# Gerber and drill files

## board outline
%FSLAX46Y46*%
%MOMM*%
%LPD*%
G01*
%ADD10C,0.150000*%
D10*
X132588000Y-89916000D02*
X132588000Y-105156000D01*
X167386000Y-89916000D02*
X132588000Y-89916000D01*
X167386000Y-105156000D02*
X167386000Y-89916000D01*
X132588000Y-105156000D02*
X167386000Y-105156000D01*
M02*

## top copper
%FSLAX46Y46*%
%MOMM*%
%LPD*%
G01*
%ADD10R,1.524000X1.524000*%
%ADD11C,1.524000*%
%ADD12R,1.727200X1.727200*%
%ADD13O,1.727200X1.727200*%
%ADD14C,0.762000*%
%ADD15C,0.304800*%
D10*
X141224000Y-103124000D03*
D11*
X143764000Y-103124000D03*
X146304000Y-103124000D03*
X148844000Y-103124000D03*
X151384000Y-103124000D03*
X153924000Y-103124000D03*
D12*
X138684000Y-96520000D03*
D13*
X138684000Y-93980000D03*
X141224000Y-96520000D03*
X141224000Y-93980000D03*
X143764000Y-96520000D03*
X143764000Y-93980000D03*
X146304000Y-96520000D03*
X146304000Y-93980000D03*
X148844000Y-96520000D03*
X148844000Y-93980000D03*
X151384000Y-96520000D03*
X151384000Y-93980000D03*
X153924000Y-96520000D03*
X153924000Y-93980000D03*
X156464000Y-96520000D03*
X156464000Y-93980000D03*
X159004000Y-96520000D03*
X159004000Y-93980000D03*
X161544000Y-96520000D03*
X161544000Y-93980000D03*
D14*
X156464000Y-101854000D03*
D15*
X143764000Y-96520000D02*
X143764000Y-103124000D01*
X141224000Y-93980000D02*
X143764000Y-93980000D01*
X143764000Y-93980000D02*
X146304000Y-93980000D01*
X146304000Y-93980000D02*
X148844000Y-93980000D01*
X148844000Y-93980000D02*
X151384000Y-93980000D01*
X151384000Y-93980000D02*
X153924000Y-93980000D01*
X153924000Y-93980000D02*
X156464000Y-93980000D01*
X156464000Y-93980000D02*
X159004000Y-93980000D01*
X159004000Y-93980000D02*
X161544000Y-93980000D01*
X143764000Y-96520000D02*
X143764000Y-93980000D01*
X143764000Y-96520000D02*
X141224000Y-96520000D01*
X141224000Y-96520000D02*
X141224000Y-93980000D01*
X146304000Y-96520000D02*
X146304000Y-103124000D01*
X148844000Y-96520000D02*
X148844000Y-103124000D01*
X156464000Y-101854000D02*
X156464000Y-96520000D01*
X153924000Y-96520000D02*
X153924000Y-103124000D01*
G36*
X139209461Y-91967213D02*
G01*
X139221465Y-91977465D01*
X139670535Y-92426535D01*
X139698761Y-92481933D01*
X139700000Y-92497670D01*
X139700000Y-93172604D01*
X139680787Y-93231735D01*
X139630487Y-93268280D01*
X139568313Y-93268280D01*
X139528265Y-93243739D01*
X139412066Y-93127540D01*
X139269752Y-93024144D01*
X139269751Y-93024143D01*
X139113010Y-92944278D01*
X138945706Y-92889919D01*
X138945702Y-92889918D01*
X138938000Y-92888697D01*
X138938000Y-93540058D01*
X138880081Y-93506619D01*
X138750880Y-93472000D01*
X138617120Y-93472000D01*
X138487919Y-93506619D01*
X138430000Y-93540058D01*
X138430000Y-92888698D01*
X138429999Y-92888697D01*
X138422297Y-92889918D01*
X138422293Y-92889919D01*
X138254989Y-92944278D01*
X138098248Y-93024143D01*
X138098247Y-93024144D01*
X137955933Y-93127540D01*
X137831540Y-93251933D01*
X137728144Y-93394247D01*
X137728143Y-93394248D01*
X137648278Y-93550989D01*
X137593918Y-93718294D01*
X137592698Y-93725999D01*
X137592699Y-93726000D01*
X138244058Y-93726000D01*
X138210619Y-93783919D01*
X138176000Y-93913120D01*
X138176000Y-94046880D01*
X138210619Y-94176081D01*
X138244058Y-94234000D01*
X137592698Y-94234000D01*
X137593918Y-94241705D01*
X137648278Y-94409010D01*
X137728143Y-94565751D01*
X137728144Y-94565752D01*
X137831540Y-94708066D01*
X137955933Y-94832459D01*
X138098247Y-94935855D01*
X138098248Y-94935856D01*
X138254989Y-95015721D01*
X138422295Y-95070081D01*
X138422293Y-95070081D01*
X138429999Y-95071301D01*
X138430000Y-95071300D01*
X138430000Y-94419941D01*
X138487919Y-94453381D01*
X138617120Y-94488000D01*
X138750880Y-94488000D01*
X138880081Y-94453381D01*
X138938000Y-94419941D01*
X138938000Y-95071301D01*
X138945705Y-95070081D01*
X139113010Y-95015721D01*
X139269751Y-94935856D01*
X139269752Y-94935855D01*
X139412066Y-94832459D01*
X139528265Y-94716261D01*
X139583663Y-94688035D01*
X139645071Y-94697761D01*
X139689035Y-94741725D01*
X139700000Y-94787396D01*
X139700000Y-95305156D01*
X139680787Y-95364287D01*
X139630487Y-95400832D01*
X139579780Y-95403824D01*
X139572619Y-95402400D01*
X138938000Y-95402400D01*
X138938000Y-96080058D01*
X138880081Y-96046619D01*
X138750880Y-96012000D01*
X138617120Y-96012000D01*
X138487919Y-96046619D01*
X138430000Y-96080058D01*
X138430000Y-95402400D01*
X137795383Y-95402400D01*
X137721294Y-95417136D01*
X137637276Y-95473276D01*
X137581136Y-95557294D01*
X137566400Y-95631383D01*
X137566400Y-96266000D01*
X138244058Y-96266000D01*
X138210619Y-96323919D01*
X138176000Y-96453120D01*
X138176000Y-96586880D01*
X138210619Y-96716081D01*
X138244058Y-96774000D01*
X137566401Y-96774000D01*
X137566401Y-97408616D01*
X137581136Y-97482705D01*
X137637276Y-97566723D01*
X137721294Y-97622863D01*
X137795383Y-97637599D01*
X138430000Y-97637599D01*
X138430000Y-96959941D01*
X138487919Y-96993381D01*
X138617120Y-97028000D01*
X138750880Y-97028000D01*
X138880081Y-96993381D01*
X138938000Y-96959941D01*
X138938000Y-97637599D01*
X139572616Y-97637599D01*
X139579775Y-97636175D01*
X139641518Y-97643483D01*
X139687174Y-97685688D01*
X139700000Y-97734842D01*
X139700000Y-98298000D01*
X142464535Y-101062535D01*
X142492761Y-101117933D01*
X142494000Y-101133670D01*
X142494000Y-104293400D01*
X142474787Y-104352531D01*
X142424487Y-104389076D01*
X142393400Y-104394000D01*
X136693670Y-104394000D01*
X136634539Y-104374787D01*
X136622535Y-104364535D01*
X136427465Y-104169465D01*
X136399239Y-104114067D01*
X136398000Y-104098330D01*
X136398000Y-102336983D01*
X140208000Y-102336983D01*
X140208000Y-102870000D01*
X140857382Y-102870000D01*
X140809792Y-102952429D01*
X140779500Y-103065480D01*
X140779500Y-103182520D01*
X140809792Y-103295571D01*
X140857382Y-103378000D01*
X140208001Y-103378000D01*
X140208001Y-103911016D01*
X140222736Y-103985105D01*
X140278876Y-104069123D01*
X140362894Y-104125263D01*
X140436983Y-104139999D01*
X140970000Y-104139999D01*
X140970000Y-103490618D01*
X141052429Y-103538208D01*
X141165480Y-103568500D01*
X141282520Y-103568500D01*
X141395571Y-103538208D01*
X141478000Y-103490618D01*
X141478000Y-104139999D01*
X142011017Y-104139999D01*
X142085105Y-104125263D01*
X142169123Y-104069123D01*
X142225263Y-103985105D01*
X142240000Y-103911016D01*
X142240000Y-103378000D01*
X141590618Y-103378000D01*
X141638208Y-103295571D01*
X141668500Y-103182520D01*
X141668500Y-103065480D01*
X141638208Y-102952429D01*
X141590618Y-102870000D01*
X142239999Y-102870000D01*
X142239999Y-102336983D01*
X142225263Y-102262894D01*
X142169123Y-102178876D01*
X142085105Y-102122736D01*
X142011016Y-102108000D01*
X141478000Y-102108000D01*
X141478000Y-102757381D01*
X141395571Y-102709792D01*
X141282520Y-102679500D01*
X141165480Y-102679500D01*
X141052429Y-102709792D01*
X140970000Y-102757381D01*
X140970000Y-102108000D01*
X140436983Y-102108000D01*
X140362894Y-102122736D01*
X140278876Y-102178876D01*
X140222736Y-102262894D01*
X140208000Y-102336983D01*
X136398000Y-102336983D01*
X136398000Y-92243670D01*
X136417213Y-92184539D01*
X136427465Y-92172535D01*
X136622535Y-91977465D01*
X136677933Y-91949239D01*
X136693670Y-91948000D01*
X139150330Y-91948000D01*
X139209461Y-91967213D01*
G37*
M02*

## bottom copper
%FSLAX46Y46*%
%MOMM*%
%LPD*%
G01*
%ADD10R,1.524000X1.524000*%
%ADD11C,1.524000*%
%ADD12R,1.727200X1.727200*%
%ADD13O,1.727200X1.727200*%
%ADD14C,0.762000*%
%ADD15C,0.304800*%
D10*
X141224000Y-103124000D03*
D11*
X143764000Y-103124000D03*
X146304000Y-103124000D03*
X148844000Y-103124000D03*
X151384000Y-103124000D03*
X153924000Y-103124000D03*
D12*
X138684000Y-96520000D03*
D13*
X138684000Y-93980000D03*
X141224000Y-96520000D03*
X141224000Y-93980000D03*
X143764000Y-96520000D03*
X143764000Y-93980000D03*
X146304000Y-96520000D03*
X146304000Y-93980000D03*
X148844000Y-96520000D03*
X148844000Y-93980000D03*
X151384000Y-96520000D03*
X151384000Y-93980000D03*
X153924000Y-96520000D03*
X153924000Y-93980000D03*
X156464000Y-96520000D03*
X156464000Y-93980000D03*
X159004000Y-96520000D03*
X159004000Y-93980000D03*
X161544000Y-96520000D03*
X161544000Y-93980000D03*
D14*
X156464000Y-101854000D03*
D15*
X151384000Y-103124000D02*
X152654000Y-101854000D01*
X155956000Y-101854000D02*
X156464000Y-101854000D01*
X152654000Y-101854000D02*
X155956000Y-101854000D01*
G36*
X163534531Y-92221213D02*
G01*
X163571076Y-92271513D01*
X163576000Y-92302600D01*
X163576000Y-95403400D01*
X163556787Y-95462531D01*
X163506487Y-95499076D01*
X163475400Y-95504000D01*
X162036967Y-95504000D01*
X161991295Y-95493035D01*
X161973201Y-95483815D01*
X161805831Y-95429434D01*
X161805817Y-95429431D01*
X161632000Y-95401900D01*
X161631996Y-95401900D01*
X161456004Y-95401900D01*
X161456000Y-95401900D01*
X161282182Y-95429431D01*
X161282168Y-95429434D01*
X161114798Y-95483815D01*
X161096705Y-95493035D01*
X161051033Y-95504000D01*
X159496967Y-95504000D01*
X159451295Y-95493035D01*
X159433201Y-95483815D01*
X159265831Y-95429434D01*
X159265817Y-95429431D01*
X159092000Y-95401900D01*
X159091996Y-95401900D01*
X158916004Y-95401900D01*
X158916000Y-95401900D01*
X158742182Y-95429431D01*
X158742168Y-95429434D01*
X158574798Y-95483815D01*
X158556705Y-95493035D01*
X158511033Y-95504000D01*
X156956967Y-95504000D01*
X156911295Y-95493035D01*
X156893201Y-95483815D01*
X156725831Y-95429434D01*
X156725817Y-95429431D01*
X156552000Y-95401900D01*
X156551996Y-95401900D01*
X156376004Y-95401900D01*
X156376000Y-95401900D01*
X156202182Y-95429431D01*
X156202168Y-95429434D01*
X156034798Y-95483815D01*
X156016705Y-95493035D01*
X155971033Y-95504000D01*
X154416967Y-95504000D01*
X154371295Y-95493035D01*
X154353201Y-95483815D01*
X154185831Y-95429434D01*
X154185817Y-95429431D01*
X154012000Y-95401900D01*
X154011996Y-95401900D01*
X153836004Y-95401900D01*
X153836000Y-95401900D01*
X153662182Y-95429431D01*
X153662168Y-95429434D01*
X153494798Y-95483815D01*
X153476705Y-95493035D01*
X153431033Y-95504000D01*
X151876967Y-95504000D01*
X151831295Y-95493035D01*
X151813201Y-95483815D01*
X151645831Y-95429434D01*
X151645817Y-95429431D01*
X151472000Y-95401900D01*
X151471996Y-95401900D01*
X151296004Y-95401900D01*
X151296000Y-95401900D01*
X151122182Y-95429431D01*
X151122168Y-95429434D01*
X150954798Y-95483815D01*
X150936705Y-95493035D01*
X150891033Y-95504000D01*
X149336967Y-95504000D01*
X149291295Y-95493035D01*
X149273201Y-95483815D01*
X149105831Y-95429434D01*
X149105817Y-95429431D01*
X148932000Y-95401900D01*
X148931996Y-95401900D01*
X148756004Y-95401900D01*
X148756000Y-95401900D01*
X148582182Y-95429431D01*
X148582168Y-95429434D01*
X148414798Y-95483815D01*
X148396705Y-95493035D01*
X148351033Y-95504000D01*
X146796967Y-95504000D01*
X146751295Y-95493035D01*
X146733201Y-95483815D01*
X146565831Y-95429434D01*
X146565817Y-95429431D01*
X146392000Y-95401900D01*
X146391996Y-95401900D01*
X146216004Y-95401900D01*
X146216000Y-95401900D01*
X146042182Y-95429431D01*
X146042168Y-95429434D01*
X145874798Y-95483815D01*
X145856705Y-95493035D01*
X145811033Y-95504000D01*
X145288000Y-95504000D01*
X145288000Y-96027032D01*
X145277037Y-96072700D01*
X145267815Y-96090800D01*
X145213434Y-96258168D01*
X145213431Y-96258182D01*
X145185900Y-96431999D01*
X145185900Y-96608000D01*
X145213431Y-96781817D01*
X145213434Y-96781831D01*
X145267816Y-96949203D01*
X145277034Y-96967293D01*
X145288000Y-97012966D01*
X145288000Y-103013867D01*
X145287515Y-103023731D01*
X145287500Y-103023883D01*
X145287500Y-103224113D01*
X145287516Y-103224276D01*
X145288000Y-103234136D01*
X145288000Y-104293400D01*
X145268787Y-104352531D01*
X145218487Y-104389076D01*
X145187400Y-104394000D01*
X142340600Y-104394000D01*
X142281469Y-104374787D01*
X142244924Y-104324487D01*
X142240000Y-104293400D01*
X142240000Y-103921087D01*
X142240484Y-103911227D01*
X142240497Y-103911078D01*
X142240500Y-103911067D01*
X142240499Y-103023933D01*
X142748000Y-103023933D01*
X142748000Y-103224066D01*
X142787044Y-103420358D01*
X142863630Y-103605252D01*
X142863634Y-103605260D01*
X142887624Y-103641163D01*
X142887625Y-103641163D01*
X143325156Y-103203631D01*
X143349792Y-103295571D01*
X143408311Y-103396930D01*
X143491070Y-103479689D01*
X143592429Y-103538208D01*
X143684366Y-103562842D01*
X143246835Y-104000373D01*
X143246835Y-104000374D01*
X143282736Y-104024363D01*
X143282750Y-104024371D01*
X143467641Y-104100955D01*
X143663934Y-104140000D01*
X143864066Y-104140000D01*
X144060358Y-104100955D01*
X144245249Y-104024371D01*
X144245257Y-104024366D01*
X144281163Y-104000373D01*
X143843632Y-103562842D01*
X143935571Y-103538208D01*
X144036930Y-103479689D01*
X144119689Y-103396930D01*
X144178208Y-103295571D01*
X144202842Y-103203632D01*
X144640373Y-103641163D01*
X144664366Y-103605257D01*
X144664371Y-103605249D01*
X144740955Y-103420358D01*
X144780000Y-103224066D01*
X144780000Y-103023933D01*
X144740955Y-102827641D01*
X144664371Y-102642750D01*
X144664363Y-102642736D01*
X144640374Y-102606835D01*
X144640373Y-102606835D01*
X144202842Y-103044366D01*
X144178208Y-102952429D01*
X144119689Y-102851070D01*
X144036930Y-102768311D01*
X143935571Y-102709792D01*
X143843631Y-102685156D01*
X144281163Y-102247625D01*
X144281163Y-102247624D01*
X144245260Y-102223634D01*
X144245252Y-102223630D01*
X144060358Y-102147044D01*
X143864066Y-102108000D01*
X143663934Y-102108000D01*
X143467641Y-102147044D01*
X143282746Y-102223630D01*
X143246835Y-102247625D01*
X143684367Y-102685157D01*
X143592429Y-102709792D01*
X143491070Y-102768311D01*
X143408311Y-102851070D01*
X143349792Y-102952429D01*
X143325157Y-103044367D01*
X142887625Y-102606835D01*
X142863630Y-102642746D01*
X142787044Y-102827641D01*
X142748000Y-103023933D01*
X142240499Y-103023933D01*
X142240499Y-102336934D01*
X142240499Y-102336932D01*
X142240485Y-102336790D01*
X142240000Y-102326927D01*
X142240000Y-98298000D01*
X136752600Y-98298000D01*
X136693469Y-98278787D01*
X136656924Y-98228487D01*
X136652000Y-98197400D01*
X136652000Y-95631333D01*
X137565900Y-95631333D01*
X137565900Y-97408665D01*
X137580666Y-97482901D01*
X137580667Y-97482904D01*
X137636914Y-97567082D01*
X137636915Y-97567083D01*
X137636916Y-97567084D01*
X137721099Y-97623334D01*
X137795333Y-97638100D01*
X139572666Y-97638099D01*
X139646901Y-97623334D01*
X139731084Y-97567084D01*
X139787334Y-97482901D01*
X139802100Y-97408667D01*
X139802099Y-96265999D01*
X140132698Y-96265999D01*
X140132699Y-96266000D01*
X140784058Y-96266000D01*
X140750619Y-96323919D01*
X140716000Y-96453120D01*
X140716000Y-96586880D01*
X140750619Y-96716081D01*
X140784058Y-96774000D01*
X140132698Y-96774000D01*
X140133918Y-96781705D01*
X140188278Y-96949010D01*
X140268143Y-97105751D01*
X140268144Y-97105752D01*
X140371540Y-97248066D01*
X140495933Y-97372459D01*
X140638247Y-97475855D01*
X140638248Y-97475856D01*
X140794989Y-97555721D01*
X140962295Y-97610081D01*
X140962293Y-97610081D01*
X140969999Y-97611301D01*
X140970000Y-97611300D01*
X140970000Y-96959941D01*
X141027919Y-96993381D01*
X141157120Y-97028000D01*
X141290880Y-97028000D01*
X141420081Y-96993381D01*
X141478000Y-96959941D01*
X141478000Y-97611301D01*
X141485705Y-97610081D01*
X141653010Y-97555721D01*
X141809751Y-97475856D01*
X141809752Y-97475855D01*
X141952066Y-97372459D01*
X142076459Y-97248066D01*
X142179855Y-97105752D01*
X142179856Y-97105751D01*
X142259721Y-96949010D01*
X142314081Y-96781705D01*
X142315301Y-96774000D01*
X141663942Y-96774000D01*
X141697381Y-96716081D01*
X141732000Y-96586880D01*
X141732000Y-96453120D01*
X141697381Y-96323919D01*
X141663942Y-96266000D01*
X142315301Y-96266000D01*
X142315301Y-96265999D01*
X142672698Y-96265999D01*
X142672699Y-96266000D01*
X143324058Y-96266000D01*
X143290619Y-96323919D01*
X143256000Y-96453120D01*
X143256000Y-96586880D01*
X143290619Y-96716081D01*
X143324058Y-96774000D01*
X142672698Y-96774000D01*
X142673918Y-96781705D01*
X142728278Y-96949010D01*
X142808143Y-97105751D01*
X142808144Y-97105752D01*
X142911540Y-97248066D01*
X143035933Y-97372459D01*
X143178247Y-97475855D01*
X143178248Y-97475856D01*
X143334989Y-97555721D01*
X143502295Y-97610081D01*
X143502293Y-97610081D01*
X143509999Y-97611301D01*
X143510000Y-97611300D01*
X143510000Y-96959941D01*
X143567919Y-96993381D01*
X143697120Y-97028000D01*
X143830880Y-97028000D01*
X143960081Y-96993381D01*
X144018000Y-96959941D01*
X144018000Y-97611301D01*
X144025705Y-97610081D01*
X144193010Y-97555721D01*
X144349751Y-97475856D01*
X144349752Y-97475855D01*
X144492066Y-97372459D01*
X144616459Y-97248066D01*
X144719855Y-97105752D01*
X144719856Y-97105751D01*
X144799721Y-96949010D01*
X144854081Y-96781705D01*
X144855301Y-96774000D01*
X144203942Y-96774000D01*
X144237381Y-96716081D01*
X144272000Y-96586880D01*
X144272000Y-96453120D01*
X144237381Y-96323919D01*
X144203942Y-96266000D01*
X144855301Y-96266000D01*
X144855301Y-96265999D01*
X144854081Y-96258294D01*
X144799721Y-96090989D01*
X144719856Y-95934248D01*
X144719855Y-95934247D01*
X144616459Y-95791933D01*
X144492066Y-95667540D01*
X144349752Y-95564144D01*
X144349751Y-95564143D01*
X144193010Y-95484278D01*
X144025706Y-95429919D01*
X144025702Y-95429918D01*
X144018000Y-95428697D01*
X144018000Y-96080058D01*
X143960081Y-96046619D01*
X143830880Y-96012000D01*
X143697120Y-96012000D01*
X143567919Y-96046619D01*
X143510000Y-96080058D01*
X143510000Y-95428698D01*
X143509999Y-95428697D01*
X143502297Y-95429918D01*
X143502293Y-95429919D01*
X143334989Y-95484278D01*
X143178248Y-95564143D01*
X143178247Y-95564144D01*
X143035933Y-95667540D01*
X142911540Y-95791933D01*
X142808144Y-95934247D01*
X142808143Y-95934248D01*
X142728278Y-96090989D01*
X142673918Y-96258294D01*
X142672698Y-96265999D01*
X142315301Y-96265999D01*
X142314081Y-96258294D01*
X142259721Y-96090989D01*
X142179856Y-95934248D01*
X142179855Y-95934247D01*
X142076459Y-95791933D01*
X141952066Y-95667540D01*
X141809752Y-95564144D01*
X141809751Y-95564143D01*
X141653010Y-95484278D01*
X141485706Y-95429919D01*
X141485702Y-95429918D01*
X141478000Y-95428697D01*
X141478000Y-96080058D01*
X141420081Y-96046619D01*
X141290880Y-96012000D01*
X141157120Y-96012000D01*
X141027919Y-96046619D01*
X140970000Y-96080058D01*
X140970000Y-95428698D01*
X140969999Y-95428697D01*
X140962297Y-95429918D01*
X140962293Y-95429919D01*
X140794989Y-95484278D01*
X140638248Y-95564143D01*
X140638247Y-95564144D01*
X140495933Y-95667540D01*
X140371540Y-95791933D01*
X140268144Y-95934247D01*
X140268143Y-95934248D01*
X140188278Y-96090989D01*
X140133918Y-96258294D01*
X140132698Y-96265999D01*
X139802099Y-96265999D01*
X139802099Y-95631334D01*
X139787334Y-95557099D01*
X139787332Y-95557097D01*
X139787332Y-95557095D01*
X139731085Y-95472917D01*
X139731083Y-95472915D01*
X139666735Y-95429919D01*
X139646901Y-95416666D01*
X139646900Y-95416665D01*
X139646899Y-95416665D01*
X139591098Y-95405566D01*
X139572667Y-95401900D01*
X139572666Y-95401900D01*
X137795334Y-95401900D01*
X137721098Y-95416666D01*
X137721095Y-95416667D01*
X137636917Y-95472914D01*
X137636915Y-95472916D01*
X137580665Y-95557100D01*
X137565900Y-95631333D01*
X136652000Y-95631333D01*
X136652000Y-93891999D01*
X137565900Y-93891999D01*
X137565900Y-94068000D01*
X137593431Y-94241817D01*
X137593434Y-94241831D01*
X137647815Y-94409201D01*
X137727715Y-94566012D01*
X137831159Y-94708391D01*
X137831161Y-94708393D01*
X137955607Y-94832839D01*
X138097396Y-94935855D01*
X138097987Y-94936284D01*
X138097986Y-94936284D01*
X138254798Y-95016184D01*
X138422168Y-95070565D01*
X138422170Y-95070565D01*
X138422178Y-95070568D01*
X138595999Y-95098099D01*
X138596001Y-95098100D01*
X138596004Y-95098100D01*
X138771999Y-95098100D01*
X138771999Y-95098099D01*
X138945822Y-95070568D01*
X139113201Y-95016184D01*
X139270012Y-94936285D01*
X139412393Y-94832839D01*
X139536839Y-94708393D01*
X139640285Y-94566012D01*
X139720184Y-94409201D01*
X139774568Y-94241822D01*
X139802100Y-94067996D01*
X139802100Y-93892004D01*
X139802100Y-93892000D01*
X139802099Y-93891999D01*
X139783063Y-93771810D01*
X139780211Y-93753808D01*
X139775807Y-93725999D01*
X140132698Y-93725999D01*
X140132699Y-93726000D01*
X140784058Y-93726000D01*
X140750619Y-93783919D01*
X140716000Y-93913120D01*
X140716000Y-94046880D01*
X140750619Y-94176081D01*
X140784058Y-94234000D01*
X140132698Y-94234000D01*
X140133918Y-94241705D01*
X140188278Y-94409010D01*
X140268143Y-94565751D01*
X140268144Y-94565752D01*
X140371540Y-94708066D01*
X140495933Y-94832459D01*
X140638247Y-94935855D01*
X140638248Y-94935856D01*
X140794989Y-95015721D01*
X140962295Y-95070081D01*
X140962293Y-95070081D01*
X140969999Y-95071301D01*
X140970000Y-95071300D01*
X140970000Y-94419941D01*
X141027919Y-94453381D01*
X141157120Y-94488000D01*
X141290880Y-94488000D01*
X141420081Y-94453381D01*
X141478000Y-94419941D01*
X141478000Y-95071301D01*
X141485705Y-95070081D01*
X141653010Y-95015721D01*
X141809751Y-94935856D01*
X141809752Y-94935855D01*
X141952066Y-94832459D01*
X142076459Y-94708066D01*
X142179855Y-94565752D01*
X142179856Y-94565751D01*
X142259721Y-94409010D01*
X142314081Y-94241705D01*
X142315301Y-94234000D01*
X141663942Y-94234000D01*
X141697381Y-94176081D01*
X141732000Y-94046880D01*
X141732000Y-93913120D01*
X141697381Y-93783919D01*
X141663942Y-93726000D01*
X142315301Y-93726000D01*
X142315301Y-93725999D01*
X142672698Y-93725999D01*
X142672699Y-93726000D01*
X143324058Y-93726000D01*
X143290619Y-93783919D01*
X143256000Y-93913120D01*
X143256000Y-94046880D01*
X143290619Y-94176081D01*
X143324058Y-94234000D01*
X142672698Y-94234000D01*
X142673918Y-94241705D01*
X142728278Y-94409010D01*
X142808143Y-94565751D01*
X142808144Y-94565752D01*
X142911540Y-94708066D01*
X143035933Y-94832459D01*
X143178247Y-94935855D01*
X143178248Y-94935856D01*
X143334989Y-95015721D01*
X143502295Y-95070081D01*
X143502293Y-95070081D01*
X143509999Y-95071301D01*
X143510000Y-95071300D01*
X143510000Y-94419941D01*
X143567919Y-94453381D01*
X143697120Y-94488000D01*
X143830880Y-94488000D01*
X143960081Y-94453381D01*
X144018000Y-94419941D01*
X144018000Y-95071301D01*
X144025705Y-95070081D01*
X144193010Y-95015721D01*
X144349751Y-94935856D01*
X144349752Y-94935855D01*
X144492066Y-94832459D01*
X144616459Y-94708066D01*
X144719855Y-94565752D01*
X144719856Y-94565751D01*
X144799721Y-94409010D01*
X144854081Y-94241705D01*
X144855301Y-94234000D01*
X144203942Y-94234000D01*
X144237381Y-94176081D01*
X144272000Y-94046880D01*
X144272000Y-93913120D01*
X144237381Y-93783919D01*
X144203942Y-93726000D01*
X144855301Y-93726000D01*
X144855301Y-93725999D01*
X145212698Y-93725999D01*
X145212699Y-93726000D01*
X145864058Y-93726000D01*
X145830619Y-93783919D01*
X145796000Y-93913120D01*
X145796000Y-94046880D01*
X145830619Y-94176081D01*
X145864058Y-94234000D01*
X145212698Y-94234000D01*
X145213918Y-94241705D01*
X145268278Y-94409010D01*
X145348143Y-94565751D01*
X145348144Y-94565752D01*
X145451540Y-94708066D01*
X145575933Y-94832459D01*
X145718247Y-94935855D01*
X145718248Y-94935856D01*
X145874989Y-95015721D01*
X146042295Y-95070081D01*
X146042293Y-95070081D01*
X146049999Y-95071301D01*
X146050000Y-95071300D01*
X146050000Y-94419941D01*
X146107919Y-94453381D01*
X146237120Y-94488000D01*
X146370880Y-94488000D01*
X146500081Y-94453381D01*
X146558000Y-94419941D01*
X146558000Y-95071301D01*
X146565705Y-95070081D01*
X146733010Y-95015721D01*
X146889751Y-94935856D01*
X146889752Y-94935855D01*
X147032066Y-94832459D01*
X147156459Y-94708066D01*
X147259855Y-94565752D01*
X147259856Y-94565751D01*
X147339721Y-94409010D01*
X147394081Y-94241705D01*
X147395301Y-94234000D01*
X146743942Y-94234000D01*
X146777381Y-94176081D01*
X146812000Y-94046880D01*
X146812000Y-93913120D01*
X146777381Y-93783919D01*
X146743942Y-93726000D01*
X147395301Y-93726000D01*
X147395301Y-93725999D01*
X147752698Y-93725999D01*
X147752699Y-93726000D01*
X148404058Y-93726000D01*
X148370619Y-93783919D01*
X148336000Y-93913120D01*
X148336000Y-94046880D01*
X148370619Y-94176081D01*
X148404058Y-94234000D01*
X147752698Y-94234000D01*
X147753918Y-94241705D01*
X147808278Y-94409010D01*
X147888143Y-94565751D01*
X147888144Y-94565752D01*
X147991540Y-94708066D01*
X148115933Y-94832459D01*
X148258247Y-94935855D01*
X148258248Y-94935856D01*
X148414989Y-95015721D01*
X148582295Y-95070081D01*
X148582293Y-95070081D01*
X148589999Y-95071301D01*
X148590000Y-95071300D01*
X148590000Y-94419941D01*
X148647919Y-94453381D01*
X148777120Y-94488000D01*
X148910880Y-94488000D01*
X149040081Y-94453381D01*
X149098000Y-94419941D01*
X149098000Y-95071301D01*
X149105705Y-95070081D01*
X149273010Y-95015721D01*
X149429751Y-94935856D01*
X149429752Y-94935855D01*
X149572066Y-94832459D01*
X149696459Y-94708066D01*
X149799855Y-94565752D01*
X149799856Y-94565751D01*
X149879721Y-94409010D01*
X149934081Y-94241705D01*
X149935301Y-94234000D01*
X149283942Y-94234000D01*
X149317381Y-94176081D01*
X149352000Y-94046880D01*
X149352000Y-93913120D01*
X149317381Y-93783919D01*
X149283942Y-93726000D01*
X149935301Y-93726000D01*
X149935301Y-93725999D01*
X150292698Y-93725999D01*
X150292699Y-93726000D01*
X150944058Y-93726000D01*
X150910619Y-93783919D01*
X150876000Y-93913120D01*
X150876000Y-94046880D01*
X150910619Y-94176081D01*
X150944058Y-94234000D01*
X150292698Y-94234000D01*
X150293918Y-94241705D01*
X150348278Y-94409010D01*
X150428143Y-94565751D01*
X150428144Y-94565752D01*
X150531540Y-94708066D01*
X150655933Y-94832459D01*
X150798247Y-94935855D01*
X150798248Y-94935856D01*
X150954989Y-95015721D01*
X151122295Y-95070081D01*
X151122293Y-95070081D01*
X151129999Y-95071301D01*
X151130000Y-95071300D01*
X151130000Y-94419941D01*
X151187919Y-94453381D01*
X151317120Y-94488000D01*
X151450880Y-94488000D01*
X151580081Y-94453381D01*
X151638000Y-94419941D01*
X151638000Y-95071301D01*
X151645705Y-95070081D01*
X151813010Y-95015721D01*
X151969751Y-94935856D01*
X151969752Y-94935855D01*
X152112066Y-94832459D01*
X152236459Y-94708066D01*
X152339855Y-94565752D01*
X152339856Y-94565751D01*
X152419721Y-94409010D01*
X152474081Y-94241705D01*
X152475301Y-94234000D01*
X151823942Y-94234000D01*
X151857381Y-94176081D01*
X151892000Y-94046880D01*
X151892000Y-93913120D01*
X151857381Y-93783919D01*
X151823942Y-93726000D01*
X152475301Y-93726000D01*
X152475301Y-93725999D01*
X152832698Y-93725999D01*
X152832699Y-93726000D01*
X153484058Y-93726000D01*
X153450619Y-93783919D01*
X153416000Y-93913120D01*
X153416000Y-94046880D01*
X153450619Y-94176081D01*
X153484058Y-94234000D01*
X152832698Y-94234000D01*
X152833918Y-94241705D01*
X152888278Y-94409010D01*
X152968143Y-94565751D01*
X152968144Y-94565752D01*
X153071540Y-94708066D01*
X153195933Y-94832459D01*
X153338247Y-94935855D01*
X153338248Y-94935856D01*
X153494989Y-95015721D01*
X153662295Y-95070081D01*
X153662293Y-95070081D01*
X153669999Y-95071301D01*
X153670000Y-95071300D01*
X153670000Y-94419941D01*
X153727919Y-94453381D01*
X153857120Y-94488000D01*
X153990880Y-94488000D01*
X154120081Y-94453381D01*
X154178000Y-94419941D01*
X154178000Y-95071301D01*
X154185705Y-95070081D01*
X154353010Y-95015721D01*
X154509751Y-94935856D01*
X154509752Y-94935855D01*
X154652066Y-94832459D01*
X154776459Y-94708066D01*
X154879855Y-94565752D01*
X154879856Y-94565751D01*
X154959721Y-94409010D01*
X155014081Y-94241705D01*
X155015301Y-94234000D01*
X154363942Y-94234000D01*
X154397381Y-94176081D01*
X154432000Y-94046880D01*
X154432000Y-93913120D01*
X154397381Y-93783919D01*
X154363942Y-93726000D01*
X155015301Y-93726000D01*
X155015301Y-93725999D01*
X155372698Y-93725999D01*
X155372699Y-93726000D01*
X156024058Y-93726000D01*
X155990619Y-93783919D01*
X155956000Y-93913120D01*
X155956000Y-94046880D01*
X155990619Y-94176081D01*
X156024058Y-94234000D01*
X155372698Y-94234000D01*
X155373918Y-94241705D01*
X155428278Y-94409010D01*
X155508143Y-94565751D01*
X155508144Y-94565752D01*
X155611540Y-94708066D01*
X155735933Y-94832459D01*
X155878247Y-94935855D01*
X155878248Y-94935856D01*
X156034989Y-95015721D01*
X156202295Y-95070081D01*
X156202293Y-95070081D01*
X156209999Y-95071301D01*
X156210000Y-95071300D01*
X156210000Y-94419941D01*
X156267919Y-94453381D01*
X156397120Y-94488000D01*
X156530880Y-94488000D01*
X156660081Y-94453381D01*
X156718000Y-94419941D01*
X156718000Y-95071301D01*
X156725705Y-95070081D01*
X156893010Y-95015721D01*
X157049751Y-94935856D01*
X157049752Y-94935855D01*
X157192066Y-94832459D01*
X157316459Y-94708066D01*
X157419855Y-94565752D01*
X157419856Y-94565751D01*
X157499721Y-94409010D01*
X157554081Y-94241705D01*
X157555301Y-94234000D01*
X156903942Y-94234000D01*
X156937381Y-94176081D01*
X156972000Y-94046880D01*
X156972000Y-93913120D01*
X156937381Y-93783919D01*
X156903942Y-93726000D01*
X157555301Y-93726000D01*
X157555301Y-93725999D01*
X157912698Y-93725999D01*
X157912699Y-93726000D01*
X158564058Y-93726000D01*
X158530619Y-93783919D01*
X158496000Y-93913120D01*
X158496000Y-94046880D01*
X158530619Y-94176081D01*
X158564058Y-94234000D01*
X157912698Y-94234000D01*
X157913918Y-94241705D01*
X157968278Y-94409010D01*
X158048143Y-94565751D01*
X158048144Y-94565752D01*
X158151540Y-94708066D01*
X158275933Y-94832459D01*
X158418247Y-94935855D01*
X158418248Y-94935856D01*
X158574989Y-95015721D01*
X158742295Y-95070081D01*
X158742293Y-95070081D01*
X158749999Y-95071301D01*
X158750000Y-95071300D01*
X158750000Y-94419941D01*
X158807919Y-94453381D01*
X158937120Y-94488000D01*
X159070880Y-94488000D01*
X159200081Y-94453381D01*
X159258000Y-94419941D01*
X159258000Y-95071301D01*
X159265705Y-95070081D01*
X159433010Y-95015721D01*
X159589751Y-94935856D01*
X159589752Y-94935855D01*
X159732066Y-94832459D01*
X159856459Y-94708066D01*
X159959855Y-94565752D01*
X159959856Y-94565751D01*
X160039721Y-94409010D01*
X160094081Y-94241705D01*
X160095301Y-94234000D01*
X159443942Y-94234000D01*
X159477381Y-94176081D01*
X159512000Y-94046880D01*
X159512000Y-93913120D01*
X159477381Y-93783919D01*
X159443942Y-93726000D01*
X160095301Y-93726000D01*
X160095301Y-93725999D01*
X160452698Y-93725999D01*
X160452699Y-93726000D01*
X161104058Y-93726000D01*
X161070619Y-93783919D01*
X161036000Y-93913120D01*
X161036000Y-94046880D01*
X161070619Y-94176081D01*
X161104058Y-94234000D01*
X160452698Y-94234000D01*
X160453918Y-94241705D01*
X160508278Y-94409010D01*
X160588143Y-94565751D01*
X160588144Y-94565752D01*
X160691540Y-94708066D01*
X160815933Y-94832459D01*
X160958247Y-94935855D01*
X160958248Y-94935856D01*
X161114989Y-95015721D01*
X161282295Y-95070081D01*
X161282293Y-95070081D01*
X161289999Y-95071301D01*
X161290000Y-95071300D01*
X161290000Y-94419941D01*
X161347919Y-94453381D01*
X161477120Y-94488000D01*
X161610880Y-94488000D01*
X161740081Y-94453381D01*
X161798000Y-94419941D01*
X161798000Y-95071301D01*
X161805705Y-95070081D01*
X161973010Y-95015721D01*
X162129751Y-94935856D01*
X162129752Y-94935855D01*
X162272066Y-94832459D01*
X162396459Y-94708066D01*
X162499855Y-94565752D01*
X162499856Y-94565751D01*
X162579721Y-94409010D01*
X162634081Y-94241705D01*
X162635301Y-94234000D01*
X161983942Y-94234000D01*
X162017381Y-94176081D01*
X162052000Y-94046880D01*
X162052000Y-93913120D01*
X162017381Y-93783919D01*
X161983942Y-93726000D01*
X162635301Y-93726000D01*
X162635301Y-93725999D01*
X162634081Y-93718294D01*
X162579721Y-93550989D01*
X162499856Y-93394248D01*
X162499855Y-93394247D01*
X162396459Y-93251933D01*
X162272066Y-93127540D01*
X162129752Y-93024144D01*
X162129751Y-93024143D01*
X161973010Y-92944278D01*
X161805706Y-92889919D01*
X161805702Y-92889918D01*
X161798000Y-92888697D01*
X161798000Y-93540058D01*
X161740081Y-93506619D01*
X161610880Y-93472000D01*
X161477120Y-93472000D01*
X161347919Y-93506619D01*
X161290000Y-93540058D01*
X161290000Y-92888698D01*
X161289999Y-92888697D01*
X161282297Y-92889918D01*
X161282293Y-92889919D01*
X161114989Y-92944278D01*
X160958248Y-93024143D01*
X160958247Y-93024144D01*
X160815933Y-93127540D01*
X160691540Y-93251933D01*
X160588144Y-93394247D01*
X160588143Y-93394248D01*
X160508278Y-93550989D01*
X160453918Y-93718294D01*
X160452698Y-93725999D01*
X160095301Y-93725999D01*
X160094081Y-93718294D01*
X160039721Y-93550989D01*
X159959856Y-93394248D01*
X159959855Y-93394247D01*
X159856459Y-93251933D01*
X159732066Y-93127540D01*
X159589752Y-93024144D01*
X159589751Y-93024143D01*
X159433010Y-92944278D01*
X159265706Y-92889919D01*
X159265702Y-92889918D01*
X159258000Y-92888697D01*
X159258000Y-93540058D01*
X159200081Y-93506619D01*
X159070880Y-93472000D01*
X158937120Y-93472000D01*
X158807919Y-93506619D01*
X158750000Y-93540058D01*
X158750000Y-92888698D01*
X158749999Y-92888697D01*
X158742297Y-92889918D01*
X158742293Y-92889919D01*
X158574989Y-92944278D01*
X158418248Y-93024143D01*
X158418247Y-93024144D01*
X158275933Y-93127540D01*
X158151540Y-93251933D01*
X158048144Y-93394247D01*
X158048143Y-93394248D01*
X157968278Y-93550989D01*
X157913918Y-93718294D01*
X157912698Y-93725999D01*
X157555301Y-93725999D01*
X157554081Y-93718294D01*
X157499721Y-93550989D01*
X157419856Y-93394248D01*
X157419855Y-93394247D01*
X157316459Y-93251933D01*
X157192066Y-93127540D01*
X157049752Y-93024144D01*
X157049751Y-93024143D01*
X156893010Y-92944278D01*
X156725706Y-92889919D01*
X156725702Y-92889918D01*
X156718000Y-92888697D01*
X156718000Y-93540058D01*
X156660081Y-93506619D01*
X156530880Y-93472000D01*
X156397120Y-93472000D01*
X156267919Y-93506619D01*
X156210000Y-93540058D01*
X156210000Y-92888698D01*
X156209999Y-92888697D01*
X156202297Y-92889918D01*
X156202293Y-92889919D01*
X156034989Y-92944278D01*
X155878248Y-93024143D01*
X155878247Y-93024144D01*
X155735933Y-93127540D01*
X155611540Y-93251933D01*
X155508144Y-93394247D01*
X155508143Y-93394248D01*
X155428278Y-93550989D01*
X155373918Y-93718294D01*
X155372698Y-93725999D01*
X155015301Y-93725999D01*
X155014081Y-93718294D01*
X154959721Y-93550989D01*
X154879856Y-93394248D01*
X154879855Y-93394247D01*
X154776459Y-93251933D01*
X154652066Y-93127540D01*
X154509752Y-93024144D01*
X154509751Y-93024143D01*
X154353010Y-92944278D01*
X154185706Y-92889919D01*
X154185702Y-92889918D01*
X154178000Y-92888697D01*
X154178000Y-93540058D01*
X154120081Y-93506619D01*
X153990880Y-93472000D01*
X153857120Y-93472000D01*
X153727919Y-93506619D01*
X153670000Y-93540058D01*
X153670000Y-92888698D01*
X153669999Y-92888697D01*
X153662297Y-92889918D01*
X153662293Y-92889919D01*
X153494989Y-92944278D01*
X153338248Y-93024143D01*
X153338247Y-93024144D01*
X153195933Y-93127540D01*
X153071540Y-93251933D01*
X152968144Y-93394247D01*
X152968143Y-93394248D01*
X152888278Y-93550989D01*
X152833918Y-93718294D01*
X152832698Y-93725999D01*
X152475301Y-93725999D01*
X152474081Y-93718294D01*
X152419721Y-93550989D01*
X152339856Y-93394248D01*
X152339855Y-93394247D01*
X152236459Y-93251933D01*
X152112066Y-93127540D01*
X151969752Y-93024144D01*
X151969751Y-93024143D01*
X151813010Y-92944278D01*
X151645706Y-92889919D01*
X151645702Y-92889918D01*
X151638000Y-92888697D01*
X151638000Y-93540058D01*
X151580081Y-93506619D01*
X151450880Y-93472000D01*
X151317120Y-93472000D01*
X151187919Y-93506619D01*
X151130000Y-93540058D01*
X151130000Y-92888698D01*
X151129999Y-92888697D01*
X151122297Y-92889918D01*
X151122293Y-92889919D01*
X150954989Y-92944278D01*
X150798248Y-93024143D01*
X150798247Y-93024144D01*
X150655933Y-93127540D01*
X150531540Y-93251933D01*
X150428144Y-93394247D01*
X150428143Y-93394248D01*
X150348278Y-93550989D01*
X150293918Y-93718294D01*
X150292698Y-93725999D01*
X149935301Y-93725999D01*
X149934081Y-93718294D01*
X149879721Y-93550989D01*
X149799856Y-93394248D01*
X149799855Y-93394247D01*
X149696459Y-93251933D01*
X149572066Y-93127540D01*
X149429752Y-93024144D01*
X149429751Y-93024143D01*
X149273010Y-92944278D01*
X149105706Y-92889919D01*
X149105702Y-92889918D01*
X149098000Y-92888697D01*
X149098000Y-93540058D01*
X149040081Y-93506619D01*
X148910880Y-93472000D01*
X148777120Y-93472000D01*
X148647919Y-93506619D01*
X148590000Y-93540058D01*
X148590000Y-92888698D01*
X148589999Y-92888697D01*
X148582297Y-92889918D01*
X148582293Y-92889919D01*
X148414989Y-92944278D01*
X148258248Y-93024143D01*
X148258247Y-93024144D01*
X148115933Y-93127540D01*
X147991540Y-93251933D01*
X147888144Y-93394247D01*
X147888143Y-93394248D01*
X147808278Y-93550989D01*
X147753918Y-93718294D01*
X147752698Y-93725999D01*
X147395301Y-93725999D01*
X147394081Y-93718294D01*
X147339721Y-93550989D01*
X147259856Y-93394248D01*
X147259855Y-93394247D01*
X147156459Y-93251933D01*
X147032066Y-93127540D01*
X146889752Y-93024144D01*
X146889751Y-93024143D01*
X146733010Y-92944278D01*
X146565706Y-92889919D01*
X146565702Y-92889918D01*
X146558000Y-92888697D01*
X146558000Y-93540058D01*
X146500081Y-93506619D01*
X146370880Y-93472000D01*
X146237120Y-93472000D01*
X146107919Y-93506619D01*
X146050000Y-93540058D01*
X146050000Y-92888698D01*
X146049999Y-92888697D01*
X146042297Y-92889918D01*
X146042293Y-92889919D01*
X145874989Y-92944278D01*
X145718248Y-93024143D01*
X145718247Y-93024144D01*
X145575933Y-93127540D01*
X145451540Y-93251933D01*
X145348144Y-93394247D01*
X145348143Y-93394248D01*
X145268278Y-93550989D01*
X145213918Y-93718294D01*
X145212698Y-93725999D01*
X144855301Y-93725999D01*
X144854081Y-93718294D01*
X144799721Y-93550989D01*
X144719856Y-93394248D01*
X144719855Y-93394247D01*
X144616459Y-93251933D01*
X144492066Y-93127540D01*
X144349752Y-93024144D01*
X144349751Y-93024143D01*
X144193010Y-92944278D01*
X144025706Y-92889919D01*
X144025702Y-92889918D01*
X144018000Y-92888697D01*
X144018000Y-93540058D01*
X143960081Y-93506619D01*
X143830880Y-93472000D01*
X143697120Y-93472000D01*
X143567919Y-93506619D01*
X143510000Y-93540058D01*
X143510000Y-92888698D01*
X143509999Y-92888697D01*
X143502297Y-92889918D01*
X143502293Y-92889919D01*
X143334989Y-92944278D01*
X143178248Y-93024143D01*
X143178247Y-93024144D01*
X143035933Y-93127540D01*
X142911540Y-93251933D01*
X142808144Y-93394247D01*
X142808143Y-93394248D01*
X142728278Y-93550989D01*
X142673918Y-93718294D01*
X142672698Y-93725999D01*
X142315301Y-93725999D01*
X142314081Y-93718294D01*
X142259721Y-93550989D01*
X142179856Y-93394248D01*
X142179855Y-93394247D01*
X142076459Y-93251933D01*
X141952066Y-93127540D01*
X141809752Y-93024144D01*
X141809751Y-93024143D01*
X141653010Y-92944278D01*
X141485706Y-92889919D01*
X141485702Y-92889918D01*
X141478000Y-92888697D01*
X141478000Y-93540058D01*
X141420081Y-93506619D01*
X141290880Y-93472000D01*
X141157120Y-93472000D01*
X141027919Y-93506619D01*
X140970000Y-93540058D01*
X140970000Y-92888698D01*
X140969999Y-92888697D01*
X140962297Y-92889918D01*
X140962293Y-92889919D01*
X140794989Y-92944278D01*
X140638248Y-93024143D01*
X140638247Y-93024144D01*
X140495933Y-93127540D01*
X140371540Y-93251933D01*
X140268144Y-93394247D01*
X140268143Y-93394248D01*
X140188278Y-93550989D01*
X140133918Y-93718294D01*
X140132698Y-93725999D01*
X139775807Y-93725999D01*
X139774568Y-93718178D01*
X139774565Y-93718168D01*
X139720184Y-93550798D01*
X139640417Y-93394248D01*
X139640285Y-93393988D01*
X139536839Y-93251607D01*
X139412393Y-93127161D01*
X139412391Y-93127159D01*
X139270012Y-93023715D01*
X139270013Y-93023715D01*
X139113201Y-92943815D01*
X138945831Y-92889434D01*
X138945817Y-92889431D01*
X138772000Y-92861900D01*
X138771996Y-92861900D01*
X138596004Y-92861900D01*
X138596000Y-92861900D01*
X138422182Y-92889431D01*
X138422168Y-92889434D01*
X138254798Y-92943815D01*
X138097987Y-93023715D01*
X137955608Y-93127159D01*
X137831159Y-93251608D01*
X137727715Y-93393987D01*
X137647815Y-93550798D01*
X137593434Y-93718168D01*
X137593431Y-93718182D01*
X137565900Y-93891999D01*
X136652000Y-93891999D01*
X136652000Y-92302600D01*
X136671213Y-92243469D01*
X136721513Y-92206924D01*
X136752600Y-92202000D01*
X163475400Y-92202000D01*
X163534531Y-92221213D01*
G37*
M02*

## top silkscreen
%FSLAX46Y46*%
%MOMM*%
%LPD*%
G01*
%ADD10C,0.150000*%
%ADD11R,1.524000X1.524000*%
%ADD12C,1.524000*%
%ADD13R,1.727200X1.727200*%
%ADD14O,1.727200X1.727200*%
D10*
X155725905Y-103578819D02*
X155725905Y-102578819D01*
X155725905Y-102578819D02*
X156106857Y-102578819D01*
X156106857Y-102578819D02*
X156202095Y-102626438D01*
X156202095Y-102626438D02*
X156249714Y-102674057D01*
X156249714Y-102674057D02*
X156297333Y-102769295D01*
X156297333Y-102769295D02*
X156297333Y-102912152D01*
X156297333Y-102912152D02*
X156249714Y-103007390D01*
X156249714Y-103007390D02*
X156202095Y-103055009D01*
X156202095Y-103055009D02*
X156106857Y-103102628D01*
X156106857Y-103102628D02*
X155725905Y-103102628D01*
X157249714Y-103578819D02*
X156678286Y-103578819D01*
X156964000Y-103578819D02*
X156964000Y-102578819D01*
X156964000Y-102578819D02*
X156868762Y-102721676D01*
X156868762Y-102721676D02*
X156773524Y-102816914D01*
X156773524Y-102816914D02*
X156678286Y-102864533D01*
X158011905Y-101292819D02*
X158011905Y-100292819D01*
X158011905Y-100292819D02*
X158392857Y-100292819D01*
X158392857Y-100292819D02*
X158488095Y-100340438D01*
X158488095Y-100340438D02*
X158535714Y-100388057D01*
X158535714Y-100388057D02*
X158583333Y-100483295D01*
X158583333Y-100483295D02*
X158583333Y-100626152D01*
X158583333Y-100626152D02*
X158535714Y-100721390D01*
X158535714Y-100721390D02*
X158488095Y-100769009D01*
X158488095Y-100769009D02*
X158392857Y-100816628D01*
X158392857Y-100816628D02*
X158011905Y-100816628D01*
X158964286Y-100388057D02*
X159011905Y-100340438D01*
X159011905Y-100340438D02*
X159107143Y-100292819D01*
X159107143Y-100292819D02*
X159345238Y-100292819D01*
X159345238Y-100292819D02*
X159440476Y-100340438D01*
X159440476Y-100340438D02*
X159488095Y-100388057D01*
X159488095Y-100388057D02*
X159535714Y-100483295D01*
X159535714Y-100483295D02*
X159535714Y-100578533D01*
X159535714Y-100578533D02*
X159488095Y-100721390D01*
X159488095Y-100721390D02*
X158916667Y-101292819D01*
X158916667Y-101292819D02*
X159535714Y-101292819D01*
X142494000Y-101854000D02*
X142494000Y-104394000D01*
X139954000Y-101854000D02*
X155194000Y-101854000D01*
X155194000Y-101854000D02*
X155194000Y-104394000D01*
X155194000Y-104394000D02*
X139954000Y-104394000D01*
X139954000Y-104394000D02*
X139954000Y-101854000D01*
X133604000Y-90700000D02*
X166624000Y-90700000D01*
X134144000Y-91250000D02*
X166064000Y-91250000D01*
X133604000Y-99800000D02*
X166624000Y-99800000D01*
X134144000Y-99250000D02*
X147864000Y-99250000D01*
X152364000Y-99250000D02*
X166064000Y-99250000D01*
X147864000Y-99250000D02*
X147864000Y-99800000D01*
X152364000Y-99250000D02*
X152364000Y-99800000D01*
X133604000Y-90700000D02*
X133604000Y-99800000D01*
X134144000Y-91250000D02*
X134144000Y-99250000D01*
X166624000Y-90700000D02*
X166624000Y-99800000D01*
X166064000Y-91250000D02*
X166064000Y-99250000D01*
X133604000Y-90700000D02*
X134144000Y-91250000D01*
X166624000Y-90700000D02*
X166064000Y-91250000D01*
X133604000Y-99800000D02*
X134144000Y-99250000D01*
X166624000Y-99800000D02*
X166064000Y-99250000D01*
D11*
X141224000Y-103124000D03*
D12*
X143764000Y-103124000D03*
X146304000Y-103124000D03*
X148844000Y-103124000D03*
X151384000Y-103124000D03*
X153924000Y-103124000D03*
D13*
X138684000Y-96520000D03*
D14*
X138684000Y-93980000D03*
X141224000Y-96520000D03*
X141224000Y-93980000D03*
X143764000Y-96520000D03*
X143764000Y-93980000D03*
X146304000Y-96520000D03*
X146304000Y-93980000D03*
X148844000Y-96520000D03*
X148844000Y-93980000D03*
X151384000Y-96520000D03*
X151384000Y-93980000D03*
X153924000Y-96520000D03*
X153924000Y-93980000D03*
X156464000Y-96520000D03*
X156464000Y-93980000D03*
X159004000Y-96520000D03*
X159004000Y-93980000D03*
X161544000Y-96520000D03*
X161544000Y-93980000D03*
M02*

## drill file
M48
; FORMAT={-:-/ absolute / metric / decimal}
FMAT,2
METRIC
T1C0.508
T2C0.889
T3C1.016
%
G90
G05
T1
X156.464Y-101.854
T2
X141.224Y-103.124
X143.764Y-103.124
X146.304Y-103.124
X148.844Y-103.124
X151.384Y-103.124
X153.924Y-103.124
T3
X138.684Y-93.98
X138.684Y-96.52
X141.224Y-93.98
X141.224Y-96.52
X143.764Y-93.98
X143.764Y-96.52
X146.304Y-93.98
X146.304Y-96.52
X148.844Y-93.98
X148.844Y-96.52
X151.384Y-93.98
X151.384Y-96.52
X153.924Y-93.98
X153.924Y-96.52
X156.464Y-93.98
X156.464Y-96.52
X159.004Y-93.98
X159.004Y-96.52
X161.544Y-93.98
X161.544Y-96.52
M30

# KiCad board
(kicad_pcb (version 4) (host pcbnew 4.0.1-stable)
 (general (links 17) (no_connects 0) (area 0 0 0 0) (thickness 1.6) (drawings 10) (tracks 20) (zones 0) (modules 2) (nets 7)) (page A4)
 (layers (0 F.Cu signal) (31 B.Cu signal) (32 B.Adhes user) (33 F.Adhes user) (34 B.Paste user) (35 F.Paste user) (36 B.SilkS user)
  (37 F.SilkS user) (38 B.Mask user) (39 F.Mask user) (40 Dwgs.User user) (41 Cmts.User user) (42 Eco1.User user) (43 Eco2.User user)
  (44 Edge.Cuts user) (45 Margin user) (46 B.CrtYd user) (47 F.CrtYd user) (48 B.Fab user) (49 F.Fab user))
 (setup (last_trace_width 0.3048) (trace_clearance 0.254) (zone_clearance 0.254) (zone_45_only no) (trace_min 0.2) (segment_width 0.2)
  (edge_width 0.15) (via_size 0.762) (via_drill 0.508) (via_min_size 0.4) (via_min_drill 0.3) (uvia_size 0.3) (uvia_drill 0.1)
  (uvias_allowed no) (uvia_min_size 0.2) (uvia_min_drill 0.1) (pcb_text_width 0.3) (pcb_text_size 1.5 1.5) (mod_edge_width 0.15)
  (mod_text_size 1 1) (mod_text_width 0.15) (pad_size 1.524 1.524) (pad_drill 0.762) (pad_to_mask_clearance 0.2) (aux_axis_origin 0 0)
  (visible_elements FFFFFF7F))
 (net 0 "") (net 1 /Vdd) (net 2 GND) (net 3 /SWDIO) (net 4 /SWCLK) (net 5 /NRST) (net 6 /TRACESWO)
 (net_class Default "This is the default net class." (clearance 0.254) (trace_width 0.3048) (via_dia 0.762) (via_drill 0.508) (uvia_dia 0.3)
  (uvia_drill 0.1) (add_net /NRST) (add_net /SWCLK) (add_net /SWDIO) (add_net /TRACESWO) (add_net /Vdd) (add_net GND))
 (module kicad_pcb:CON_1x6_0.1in (layer F.Cu) (at 147.574 103.124)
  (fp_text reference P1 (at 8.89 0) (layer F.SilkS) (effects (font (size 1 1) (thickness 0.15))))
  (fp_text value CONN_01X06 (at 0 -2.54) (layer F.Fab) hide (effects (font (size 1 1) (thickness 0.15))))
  (fp_line (start -5.08 -1.27) (end -5.08 1.27) (layer F.SilkS) (width 0.15))
  (fp_line (start -7.62 -1.27) (end 7.62 -1.27) (layer F.SilkS) (width 0.15))
  (fp_line (start 7.62 -1.27) (end 7.62 1.27) (layer F.SilkS) (width 0.15))
  (fp_line (start 7.62 1.27) (end -7.62 1.27) (layer F.SilkS) (width 0.15))
  (fp_line (start -7.62 1.27) (end -7.62 -1.27) (layer F.SilkS) (width 0.15))
  (pad 1 thru_hole rect (at -6.35 0) (size 1.524 1.524) (drill 0.889) (layers *.Cu *.Mask F.SilkS) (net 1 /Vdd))
  (pad 2 thru_hole circle (at -3.81 0) (size 1.524 1.524) (drill 0.889) (layers *.Cu *.Mask F.SilkS) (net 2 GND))
  (pad 3 thru_hole circle (at -1.27 0) (size 1.524 1.524) (drill 0.889) (layers *.Cu *.Mask F.SilkS) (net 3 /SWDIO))
  (pad 4 thru_hole circle (at 1.27 0) (size 1.524 1.524) (drill 0.889) (layers *.Cu *.Mask F.SilkS) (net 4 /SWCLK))
  (pad 5 thru_hole circle (at 3.81 0) (size 1.524 1.524) (drill 0.889) (layers *.Cu *.Mask F.SilkS) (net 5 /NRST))
  (pad 6 thru_hole circle (at 6.35 0) (size 1.524 1.524) (drill 0.889) (layers *.Cu *.Mask F.SilkS) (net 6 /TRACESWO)))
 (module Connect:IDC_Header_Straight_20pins (layer F.Cu) (at 138.684 96.52)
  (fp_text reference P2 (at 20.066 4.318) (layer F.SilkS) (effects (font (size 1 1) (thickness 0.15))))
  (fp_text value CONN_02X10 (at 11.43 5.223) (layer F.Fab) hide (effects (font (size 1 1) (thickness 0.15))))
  (fp_line (start -5.08 -5.82) (end 27.94 -5.82) (layer F.SilkS) (width 0.15))
  (fp_line (start -4.54 -5.27) (end 27.38 -5.27) (layer F.SilkS) (width 0.15))
  (fp_line (start -5.08 3.28) (end 27.94 3.28) (layer F.SilkS) (width 0.15))
  (fp_line (start -4.54 2.73) (end 9.18 2.73) (layer F.SilkS) (width 0.15))
  (fp_line (start 13.68 2.73) (end 27.38 2.73) (layer F.SilkS) (width 0.15))
  (fp_line (start 9.18 2.73) (end 9.18 3.28) (layer F.SilkS) (width 0.15))
  (fp_line (start 13.68 2.73) (end 13.68 3.28) (layer F.SilkS) (width 0.15))
  (fp_line (start -5.08 -5.82) (end -5.08 3.28) (layer F.SilkS) (width 0.15))
  (fp_line (start -4.54 -5.27) (end -4.54 2.73) (layer F.SilkS) (width 0.15))
  (fp_line (start 27.94 -5.82) (end 27.94 3.28) (layer F.SilkS) (width 0.15))
  (fp_line (start 27.38 -5.27) (end 27.38 2.73) (layer F.SilkS) (width 0.15))
  (fp_line (start -5.08 -5.82) (end -4.54 -5.27) (layer F.SilkS) (width 0.15))
  (fp_line (start 27.94 -5.82) (end 27.38 -5.27) (layer F.SilkS) (width 0.15))
  (fp_line (start -5.08 3.28) (end -4.54 2.73) (layer F.SilkS) (width 0.15))
  (fp_line (start 27.94 3.28) (end 27.38 2.73) (layer F.SilkS) (width 0.15))
  (pad 1 thru_hole rect (at 0 0) (size 1.7272 1.7272) (drill 1.016) (layers *.Cu *.Mask F.SilkS) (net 1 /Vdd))
  (pad 2 thru_hole oval (at 0 -2.54) (size 1.7272 1.7272) (drill 1.016) (layers *.Cu *.Mask F.SilkS) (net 1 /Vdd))
  (pad 3 thru_hole oval (at 2.54 0) (size 1.7272 1.7272) (drill 1.016) (layers *.Cu *.Mask F.SilkS) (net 2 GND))
  (pad 4 thru_hole oval (at 2.54 -2.54) (size 1.7272 1.7272) (drill 1.016) (layers *.Cu *.Mask F.SilkS) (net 2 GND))
  (pad 5 thru_hole oval (at 5.08 0) (size 1.7272 1.7272) (drill 1.016) (layers *.Cu *.Mask F.SilkS) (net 2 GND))
  (pad 6 thru_hole oval (at 5.08 -2.54) (size 1.7272 1.7272) (drill 1.016) (layers *.Cu *.Mask F.SilkS) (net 2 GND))
  (pad 7 thru_hole oval (at 7.62 0) (size 1.7272 1.7272) (drill 1.016) (layers *.Cu *.Mask F.SilkS) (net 3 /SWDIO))
  (pad 8 thru_hole oval (at 7.62 -2.54) (size 1.7272 1.7272) (drill 1.016) (layers *.Cu *.Mask F.SilkS) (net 2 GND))
  (pad 9 thru_hole oval (at 10.16 0) (size 1.7272 1.7272) (drill 1.016) (layers *.Cu *.Mask F.SilkS) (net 4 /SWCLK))
  (pad 10 thru_hole oval (at 10.16 -2.54) (size 1.7272 1.7272) (drill 1.016) (layers *.Cu *.Mask F.SilkS) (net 2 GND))
  (pad 11 thru_hole oval (at 12.7 0) (size 1.7272 1.7272) (drill 1.016) (layers *.Cu *.Mask F.SilkS))
  (pad 12 thru_hole oval (at 12.7 -2.54) (size 1.7272 1.7272) (drill 1.016) (layers *.Cu *.Mask F.SilkS) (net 2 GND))
  (pad 13 thru_hole oval (at 15.24 0) (size 1.7272 1.7272) (drill 1.016) (layers *.Cu *.Mask F.SilkS) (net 6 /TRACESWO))
  (pad 14 thru_hole oval (at 15.24 -2.54) (size 1.7272 1.7272) (drill 1.016) (layers *.Cu *.Mask F.SilkS) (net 2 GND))
  (pad 15 thru_hole oval (at 17.78 0) (size 1.7272 1.7272) (drill 1.016) (layers *.Cu *.Mask F.SilkS) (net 5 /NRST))
  (pad 16 thru_hole oval (at 17.78 -2.54) (size 1.7272 1.7272) (drill 1.016) (layers *.Cu *.Mask F.SilkS) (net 2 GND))
  (pad 17 thru_hole oval (at 20.32 0) (size 1.7272 1.7272) (drill 1.016) (layers *.Cu *.Mask F.SilkS))
  (pad 18 thru_hole oval (at 20.32 -2.54) (size 1.7272 1.7272) (drill 1.016) (layers *.Cu *.Mask F.SilkS) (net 2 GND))
  (pad 19 thru_hole oval (at 22.86 0) (size 1.7272 1.7272) (drill 1.016) (layers *.Cu *.Mask F.SilkS))
  (pad 20 thru_hole oval (at 22.86 -2.54) (size 1.7272 1.7272) (drill 1.016) (layers *.Cu *.Mask F.SilkS) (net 2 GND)))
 (gr_line (start 132.588 89.916) (end 132.588 105.156) (angle 90) (layer Edge.Cuts) (width 0.15))
 (gr_line (start 167.386 89.916) (end 132.588 89.916) (angle 90) (layer Edge.Cuts) (width 0.15))
 (gr_line (start 167.386 105.156) (end 167.386 89.916) (angle 90) (layer Edge.Cuts) (width 0.15))
 (gr_line (start 132.588 105.156) (end 167.386 105.156) (angle 90) (layer Edge.Cuts) (width 0.15))
 (segment (start 143.764 96.52) (end 143.764 103.124) (width 0.3048) (layer F.Cu) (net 2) (status C00000))
 (segment (start 141.224 93.98) (end 143.764 93.98) (width 0.3048) (layer F.Cu) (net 2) (status C00000))
 (segment (start 143.764 93.98) (end 146.304 93.98) (width 0.3048) (layer F.Cu) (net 2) (status C00000))
 (segment (start 146.304 93.98) (end 148.844 93.98) (width 0.3048) (layer F.Cu) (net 2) (status C00000))
 (segment (start 148.844 93.98) (end 151.384 93.98) (width 0.3048) (layer F.Cu) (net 2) (status C00000))
 (segment (start 151.384 93.98) (end 153.924 93.98) (width 0.3048) (layer F.Cu) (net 2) (status C00000))
 (segment (start 153.924 93.98) (end 156.464 93.98) (width 0.3048) (layer F.Cu) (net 2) (status C00000))
 (segment (start 156.464 93.98) (end 159.004 93.98) (width 0.3048) (layer F.Cu) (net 2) (status C00000))
 (segment (start 159.004 93.98) (end 161.544 93.98) (width 0.3048) (layer F.Cu) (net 2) (status C00000))
 (segment (start 143.764 96.52) (end 143.764 93.98) (width 0.3048) (layer F.Cu) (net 2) (status C00000))
 (segment (start 143.764 96.52) (end 141.224 96.52) (width 0.3048) (layer F.Cu) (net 2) (status C00000))
 (segment (start 141.224 96.52) (end 141.224 93.98) (width 0.3048) (layer F.Cu) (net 2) (status C00000))
 (segment (start 146.304 96.52) (end 146.304 103.124) (width 0.3048) (layer F.Cu) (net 3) (status C00000))
 (segment (start 148.844 96.52) (end 148.844 103.124) (width 0.3048) (layer F.Cu) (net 4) (status C00000))
 (segment (start 151.384 103.124) (end 152.654 101.854) (width 0.3048) (layer B.Cu) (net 5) (status 400000))
 (segment (start 156.464 101.854) (end 156.464 96.52) (width 0.3048) (layer F.Cu) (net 5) (status 800000))
 (via (at 156.464 101.854) (size 0.762) (drill 0.508) (layers F.Cu B.Cu) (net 5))
 (segment (start 155.956 101.854) (end 156.464 101.854) (width 0.3048) (layer B.Cu) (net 5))
 (segment (start 152.654 101.854) (end 155.956 101.854) (width 0.3048) (layer B.Cu) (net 5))
 (segment (start 153.924 96.52) (end 153.924 103.124) (width 0.3048) (layer F.Cu) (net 6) (status C00000))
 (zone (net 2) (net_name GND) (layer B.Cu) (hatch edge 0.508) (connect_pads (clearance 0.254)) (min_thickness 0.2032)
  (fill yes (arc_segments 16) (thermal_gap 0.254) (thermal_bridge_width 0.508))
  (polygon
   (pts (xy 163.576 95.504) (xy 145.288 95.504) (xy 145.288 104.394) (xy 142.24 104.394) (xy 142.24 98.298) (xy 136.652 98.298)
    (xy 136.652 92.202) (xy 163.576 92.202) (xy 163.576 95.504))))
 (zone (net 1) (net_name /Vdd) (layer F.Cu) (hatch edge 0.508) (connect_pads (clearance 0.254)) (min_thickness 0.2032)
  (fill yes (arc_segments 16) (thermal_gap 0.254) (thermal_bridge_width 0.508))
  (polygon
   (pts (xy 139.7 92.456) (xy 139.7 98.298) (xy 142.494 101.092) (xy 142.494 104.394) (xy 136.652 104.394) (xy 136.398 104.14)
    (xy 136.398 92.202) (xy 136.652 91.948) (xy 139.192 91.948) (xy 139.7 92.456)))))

